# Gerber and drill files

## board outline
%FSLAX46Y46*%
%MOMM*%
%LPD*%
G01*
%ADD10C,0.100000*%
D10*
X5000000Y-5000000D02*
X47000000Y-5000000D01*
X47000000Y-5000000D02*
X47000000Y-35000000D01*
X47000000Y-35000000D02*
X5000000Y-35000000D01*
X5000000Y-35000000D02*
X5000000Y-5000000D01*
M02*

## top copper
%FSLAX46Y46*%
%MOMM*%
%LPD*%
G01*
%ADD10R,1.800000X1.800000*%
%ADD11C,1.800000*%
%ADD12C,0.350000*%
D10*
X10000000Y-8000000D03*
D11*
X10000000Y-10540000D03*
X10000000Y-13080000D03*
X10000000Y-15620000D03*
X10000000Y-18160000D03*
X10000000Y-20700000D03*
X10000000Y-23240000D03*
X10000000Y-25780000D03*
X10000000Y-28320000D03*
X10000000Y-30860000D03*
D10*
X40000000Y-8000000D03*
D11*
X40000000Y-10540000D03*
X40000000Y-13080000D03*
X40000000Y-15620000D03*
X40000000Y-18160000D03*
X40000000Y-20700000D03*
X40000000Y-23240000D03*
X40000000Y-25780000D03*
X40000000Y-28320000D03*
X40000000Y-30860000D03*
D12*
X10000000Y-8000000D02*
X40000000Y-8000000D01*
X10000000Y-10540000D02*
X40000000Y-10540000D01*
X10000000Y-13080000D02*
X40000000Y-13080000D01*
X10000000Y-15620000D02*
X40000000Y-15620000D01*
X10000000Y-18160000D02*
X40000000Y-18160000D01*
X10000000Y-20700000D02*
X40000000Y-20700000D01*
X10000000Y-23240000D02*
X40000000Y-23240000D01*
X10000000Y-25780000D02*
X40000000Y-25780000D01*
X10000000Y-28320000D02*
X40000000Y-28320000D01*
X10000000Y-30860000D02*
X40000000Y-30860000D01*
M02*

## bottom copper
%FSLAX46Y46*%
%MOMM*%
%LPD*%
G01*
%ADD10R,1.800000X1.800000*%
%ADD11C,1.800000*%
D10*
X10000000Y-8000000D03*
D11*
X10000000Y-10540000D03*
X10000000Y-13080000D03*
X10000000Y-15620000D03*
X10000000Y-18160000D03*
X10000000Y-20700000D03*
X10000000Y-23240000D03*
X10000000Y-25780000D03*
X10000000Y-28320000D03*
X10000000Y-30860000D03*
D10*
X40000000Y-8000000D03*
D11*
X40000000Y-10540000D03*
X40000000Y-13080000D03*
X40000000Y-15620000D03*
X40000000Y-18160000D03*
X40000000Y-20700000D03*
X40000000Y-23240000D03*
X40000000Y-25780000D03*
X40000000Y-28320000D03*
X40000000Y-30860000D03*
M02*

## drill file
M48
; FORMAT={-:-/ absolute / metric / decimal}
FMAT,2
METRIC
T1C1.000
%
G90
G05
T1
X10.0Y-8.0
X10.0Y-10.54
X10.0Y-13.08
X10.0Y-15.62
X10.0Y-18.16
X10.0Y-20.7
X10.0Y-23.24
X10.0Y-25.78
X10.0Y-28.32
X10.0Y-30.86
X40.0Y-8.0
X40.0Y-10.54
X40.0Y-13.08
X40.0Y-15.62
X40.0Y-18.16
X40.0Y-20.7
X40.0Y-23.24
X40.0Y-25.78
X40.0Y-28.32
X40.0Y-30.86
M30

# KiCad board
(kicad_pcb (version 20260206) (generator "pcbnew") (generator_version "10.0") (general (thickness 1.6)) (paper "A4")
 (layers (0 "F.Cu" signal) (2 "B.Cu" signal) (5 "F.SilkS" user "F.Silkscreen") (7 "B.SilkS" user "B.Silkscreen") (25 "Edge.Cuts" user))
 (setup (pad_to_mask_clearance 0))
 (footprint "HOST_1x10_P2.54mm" (layer "F.Cu") (at 10 8)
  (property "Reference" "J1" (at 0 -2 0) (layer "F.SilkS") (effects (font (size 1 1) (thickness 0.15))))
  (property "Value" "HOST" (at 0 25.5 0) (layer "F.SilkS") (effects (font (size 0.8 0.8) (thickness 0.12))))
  (pad "1" thru_hole rect (at 0 0) (size 1.8 1.8) (drill 1) (layers "*.Cu" "*.Mask") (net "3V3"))
  (pad "2" thru_hole circle (at 0 2.54) (size 1.8 1.8) (drill 1) (layers "*.Cu" "*.Mask") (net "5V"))
  (pad "3" thru_hole circle (at 0 5.08) (size 1.8 1.8) (drill 1) (layers "*.Cu" "*.Mask") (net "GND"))
  (pad "4" thru_hole circle (at 0 7.62) (size 1.8 1.8) (drill 1) (layers "*.Cu" "*.Mask") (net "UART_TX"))
  (pad "5" thru_hole circle (at 0 10.16) (size 1.8 1.8) (drill 1) (layers "*.Cu" "*.Mask") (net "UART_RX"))
  (pad "6" thru_hole circle (at 0 12.7) (size 1.8 1.8) (drill 1) (layers "*.Cu" "*.Mask") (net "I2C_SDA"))
  (pad "7" thru_hole circle (at 0 15.24) (size 1.8 1.8) (drill 1) (layers "*.Cu" "*.Mask") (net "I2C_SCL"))
  (pad "8" thru_hole circle (at 0 17.78) (size 1.8 1.8) (drill 1) (layers "*.Cu" "*.Mask") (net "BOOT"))
  (pad "9" thru_hole circle (at 0 20.32) (size 1.8 1.8) (drill 1) (layers "*.Cu" "*.Mask") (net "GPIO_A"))
  (pad "10" thru_hole circle (at 0 22.86) (size 1.8 1.8) (drill 1) (layers "*.Cu" "*.Mask") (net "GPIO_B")))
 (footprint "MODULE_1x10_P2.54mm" (layer "F.Cu") (at 40 8)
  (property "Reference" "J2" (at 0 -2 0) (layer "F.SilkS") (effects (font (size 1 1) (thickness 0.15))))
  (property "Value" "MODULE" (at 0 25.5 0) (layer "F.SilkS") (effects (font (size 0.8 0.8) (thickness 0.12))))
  (pad "1" thru_hole rect (at 0 0) (size 1.8 1.8) (drill 1) (layers "*.Cu" "*.Mask") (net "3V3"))
  (pad "2" thru_hole circle (at 0 2.54) (size 1.8 1.8) (drill 1) (layers "*.Cu" "*.Mask") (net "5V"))
  (pad "3" thru_hole circle (at 0 5.08) (size 1.8 1.8) (drill 1) (layers "*.Cu" "*.Mask") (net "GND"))
  (pad "4" thru_hole circle (at 0 7.62) (size 1.8 1.8) (drill 1) (layers "*.Cu" "*.Mask") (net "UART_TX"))
  (pad "5" thru_hole circle (at 0 10.16) (size 1.8 1.8) (drill 1) (layers "*.Cu" "*.Mask") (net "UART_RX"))
  (pad "6" thru_hole circle (at 0 12.7) (size 1.8 1.8) (drill 1) (layers "*.Cu" "*.Mask") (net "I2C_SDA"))
  (pad "7" thru_hole circle (at 0 15.24) (size 1.8 1.8) (drill 1) (layers "*.Cu" "*.Mask") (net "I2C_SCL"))
  (pad "8" thru_hole circle (at 0 17.78) (size 1.8 1.8) (drill 1) (layers "*.Cu" "*.Mask") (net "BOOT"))
  (pad "9" thru_hole circle (at 0 20.32) (size 1.8 1.8) (drill 1) (layers "*.Cu" "*.Mask") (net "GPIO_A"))
  (pad "10" thru_hole circle (at 0 22.86) (size 1.8 1.8) (drill 1) (layers "*.Cu" "*.Mask") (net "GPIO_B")))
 (gr_line (start 5 5) (end 47 5) (stroke (width 0.1) (type default)) (layer "Edge.Cuts"))
 (gr_line (start 47 5) (end 47 35) (stroke (width 0.1) (type default)) (layer "Edge.Cuts"))
 (gr_line (start 47 35) (end 5 35) (stroke (width 0.1) (type default)) (layer "Edge.Cuts"))
 (gr_line (start 5 35) (end 5 5) (stroke (width 0.1) (type default)) (layer "Edge.Cuts"))
 (segment (start 10 8) (end 40 8) (width 0.35) (layer "F.Cu") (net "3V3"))
 (segment (start 10 10.54) (end 40 10.54) (width 0.35) (layer "F.Cu") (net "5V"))
 (segment (start 10 13.08) (end 40 13.08) (width 0.35) (layer "F.Cu") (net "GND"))
 (segment (start 10 15.62) (end 40 15.62) (width 0.35) (layer "F.Cu") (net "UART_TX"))
 (segment (start 10 18.16) (end 40 18.16) (width 0.35) (layer "F.Cu") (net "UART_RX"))
 (segment (start 10 20.7) (end 40 20.7) (width 0.35) (layer "F.Cu") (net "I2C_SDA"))
 (segment (start 10 23.24) (end 40 23.24) (width 0.35) (layer "F.Cu") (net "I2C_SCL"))
 (segment (start 10 25.78) (end 40 25.78) (width 0.35) (layer "F.Cu") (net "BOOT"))
 (segment (start 10 28.32) (end 40 28.32) (width 0.35) (layer "F.Cu") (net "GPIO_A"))
 (segment (start 10 30.86) (end 40 30.86) (width 0.35) (layer "F.Cu") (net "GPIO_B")))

